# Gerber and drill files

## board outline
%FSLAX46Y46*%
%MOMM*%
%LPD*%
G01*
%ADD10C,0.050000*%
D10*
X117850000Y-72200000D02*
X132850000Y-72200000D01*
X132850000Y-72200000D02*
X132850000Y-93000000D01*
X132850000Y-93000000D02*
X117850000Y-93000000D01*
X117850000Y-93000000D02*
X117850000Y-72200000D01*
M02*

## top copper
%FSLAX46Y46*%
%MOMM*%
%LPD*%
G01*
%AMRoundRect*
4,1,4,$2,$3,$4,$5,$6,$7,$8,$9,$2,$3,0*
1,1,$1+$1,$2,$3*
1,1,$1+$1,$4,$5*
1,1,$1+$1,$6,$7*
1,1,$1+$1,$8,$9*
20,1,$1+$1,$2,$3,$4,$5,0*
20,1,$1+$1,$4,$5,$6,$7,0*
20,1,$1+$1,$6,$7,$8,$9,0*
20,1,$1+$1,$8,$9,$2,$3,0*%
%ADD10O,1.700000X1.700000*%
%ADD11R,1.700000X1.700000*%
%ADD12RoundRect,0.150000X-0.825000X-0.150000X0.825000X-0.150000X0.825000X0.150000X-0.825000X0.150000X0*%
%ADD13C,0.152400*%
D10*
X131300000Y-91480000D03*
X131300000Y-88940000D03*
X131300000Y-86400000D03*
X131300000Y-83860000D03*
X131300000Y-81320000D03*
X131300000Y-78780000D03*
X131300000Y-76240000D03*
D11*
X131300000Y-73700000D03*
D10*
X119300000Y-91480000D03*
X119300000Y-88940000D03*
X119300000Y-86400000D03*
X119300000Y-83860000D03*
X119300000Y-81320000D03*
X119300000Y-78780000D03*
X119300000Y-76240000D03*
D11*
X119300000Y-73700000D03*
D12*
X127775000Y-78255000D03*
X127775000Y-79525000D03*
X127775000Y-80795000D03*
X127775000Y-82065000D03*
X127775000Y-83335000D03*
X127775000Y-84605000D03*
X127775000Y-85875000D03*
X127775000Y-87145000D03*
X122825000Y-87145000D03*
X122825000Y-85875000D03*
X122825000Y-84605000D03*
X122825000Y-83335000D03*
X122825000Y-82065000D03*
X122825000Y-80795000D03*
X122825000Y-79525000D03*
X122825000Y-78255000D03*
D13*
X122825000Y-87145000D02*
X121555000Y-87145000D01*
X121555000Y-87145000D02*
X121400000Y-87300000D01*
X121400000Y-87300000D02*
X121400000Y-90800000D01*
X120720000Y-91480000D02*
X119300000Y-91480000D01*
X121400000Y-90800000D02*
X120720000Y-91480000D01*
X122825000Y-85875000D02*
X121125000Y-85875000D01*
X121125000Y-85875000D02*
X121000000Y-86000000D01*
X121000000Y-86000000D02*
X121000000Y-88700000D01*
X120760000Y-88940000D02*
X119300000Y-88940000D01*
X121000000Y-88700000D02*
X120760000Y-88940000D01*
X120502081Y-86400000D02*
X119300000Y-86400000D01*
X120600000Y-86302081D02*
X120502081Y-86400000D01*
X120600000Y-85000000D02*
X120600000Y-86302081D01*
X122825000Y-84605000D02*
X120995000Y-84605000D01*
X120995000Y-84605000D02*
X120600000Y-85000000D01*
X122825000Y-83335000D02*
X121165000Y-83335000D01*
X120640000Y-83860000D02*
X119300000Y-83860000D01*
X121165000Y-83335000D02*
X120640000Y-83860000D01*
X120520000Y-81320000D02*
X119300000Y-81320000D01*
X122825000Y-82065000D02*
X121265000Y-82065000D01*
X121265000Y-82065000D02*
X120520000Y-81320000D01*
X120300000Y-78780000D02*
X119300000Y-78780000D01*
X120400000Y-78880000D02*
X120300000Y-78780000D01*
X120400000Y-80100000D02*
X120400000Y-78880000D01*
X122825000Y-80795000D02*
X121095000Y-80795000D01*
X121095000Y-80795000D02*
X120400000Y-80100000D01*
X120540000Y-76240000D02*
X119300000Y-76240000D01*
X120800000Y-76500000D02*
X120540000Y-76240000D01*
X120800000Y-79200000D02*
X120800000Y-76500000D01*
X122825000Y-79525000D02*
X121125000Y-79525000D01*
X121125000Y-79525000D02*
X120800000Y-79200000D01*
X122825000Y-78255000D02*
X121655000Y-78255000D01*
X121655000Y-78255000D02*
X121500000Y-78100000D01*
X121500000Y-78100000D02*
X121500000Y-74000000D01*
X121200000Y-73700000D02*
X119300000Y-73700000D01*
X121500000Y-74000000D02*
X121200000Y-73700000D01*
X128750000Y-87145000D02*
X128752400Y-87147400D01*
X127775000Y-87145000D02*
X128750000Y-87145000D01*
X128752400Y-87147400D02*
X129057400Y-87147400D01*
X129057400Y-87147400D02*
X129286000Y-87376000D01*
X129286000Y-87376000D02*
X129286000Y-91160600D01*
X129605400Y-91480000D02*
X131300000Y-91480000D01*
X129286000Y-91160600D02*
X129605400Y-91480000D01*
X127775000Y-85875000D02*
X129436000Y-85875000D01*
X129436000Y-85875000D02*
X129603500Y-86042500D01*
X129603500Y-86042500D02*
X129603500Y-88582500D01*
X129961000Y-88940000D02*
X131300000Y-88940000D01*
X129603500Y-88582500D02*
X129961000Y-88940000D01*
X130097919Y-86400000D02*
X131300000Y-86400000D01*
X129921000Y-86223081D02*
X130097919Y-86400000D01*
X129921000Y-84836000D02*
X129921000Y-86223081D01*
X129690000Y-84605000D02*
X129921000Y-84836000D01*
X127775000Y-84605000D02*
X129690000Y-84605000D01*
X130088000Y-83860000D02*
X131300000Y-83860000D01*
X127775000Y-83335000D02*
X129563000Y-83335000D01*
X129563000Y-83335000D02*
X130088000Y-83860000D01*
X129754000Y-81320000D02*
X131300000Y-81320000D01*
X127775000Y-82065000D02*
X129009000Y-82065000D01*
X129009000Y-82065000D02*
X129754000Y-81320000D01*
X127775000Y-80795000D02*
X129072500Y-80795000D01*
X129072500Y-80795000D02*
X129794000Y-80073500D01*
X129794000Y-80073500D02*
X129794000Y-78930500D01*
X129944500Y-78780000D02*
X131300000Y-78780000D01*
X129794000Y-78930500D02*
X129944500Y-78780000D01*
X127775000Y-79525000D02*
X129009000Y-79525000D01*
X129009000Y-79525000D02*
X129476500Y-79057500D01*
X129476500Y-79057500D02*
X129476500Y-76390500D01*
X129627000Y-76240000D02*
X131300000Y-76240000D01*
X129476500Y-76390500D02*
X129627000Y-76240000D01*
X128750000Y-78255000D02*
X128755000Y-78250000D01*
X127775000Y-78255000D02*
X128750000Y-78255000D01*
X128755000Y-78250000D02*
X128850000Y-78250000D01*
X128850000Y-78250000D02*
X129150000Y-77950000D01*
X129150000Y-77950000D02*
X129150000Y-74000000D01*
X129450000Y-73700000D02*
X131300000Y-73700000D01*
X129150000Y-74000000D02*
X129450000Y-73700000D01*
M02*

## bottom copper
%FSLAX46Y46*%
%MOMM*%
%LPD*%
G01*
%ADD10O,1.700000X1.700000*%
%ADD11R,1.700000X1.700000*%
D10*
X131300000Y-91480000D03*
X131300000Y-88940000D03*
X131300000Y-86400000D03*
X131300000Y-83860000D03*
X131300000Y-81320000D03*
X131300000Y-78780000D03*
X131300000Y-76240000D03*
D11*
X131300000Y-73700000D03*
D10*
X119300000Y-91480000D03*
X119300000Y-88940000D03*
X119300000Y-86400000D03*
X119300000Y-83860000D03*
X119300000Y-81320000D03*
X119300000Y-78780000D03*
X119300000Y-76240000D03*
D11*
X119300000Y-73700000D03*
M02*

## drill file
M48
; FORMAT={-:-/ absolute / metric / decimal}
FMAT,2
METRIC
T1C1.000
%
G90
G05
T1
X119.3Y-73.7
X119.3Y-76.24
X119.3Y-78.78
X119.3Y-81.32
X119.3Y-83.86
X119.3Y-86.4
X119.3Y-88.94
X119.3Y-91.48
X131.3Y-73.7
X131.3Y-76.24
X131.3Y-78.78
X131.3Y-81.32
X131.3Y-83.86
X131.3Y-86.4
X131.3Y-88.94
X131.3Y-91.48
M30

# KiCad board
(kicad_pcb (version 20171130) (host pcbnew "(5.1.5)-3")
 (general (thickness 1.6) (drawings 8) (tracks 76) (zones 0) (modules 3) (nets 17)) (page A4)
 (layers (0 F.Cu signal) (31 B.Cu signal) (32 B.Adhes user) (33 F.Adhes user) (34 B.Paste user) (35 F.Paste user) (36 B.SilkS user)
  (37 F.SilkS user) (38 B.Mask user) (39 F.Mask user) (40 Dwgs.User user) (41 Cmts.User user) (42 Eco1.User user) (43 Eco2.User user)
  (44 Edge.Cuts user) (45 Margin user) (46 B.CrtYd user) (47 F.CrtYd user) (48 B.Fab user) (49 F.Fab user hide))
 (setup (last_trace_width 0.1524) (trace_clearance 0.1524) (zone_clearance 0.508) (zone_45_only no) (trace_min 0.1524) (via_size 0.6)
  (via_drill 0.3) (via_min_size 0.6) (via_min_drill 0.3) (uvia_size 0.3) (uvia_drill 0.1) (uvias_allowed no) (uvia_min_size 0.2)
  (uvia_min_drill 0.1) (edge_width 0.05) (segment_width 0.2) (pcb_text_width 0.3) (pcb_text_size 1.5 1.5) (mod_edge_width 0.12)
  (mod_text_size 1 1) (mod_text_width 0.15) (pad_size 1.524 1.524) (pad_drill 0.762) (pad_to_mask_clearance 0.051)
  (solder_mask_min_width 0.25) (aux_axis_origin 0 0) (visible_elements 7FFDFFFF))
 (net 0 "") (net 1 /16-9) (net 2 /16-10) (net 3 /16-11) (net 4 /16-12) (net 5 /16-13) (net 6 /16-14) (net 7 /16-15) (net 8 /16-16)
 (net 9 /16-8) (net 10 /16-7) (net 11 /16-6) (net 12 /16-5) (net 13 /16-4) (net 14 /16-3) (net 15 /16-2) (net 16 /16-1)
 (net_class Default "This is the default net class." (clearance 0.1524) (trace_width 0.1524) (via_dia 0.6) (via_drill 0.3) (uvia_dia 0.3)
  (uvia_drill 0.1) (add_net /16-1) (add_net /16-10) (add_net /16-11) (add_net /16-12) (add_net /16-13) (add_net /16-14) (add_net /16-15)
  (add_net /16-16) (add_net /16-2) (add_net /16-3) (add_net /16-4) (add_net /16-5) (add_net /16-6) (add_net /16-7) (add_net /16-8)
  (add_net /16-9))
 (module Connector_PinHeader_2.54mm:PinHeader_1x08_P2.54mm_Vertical (layer F.Cu) (at 131.3 73.7)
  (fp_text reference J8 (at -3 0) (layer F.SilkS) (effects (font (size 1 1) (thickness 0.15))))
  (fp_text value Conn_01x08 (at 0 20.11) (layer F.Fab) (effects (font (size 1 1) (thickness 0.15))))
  (pad 8 thru_hole oval (at 0 17.78) (size 1.7 1.7) (drill 1) (layers *.Cu *.Mask) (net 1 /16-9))
  (pad 7 thru_hole oval (at 0 15.24) (size 1.7 1.7) (drill 1) (layers *.Cu *.Mask) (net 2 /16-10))
  (pad 6 thru_hole oval (at 0 12.7) (size 1.7 1.7) (drill 1) (layers *.Cu *.Mask) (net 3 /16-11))
  (pad 5 thru_hole oval (at 0 10.16) (size 1.7 1.7) (drill 1) (layers *.Cu *.Mask) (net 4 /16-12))
  (pad 4 thru_hole oval (at 0 7.62) (size 1.7 1.7) (drill 1) (layers *.Cu *.Mask) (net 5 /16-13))
  (pad 3 thru_hole oval (at 0 5.08) (size 1.7 1.7) (drill 1) (layers *.Cu *.Mask) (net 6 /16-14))
  (pad 2 thru_hole oval (at 0 2.54) (size 1.7 1.7) (drill 1) (layers *.Cu *.Mask) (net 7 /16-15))
  (pad 1 thru_hole rect (at 0 0) (size 1.7 1.7) (drill 1) (layers *.Cu *.Mask) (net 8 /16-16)))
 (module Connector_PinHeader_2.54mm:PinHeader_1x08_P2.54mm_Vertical (layer F.Cu) (at 119.3 73.7)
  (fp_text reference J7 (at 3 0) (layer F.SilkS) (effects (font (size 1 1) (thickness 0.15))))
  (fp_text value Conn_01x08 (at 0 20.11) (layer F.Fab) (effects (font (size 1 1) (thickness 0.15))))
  (pad 8 thru_hole oval (at 0 17.78) (size 1.7 1.7) (drill 1) (layers *.Cu *.Mask) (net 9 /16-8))
  (pad 7 thru_hole oval (at 0 15.24) (size 1.7 1.7) (drill 1) (layers *.Cu *.Mask) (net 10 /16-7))
  (pad 6 thru_hole oval (at 0 12.7) (size 1.7 1.7) (drill 1) (layers *.Cu *.Mask) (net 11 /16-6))
  (pad 5 thru_hole oval (at 0 10.16) (size 1.7 1.7) (drill 1) (layers *.Cu *.Mask) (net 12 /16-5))
  (pad 4 thru_hole oval (at 0 7.62) (size 1.7 1.7) (drill 1) (layers *.Cu *.Mask) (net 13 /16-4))
  (pad 3 thru_hole oval (at 0 5.08) (size 1.7 1.7) (drill 1) (layers *.Cu *.Mask) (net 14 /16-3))
  (pad 2 thru_hole oval (at 0 2.54) (size 1.7 1.7) (drill 1) (layers *.Cu *.Mask) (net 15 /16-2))
  (pad 1 thru_hole rect (at 0 0) (size 1.7 1.7) (drill 1) (layers *.Cu *.Mask) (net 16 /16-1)))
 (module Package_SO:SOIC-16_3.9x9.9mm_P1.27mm (layer F.Cu) (at 125.3 82.7)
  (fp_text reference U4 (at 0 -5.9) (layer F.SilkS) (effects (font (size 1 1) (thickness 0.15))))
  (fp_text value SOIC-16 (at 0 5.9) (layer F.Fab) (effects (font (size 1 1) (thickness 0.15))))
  (pad 16 smd roundrect (at 2.475 -4.445) (size 1.95 0.6) (layers F.Cu F.Paste F.Mask) (roundrect_rratio 0.25) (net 8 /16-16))
  (pad 15 smd roundrect (at 2.475 -3.175) (size 1.95 0.6) (layers F.Cu F.Paste F.Mask) (roundrect_rratio 0.25) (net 7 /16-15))
  (pad 14 smd roundrect (at 2.475 -1.905) (size 1.95 0.6) (layers F.Cu F.Paste F.Mask) (roundrect_rratio 0.25) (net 6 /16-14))
  (pad 13 smd roundrect (at 2.475 -0.635) (size 1.95 0.6) (layers F.Cu F.Paste F.Mask) (roundrect_rratio 0.25) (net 5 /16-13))
  (pad 12 smd roundrect (at 2.475 0.635) (size 1.95 0.6) (layers F.Cu F.Paste F.Mask) (roundrect_rratio 0.25) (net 4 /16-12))
  (pad 11 smd roundrect (at 2.475 1.905) (size 1.95 0.6) (layers F.Cu F.Paste F.Mask) (roundrect_rratio 0.25) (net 3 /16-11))
  (pad 10 smd roundrect (at 2.475 3.175) (size 1.95 0.6) (layers F.Cu F.Paste F.Mask) (roundrect_rratio 0.25) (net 2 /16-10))
  (pad 9 smd roundrect (at 2.475 4.445) (size 1.95 0.6) (layers F.Cu F.Paste F.Mask) (roundrect_rratio 0.25) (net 1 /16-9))
  (pad 8 smd roundrect (at -2.475 4.445) (size 1.95 0.6) (layers F.Cu F.Paste F.Mask) (roundrect_rratio 0.25) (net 9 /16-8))
  (pad 7 smd roundrect (at -2.475 3.175) (size 1.95 0.6) (layers F.Cu F.Paste F.Mask) (roundrect_rratio 0.25) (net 10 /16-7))
  (pad 6 smd roundrect (at -2.475 1.905) (size 1.95 0.6) (layers F.Cu F.Paste F.Mask) (roundrect_rratio 0.25) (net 11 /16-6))
  (pad 5 smd roundrect (at -2.475 0.635) (size 1.95 0.6) (layers F.Cu F.Paste F.Mask) (roundrect_rratio 0.25) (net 12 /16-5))
  (pad 4 smd roundrect (at -2.475 -0.635) (size 1.95 0.6) (layers F.Cu F.Paste F.Mask) (roundrect_rratio 0.25) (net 13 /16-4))
  (pad 3 smd roundrect (at -2.475 -1.905) (size 1.95 0.6) (layers F.Cu F.Paste F.Mask) (roundrect_rratio 0.25) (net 14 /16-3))
  (pad 2 smd roundrect (at -2.475 -3.175) (size 1.95 0.6) (layers F.Cu F.Paste F.Mask) (roundrect_rratio 0.25) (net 15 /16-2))
  (pad 1 smd roundrect (at -2.475 -4.445) (size 1.95 0.6) (layers F.Cu F.Paste F.Mask) (roundrect_rratio 0.25) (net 16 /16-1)))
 (gr_line (start 117.85 72.2) (end 132.85 72.2) (layer Edge.Cuts) (width 0.05))
 (gr_line (start 132.85 72.2) (end 132.85 93) (layer Edge.Cuts) (width 0.05))
 (gr_line (start 132.85 93) (end 117.85 93) (layer Edge.Cuts) (width 0.05))
 (gr_line (start 117.85 93) (end 117.85 72.2) (layer Edge.Cuts) (width 0.05))
 (segment (start 122.825 87.145) (end 121.555 87.145) (width 0.1524) (layer F.Cu) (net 9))
 (segment (start 121.555 87.145) (end 121.4 87.3) (width 0.1524) (layer F.Cu) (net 9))
 (segment (start 121.4 87.3) (end 121.4 90.8) (width 0.1524) (layer F.Cu) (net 9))
 (segment (start 120.72 91.48) (end 119.3 91.48) (width 0.1524) (layer F.Cu) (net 9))
 (segment (start 121.4 90.8) (end 120.72 91.48) (width 0.1524) (layer F.Cu) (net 9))
 (segment (start 122.825 85.875) (end 121.125 85.875) (width 0.1524) (layer F.Cu) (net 10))
 (segment (start 121.125 85.875) (end 121 86) (width 0.1524) (layer F.Cu) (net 10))
 (segment (start 121 86) (end 121 88.7) (width 0.1524) (layer F.Cu) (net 10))
 (segment (start 120.76 88.94) (end 119.3 88.94) (width 0.1524) (layer F.Cu) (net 10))
 (segment (start 121 88.7) (end 120.76 88.94) (width 0.1524) (layer F.Cu) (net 10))
 (segment (start 120.502081 86.4) (end 119.3 86.4) (width 0.1524) (layer F.Cu) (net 11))
 (segment (start 120.6 86.302081) (end 120.502081 86.4) (width 0.1524) (layer F.Cu) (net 11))
 (segment (start 120.6 85) (end 120.6 86.302081) (width 0.1524) (layer F.Cu) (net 11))
 (segment (start 122.825 84.605) (end 120.995 84.605) (width 0.1524) (layer F.Cu) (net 11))
 (segment (start 120.995 84.605) (end 120.6 85) (width 0.1524) (layer F.Cu) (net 11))
 (segment (start 122.825 83.335) (end 121.165 83.335) (width 0.1524) (layer F.Cu) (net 12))
 (segment (start 120.64 83.86) (end 119.3 83.86) (width 0.1524) (layer F.Cu) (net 12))
 (segment (start 121.165 83.335) (end 120.64 83.86) (width 0.1524) (layer F.Cu) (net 12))
 (segment (start 120.52 81.32) (end 119.3 81.32) (width 0.1524) (layer F.Cu) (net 13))
 (segment (start 122.825 82.065) (end 121.265 82.065) (width 0.1524) (layer F.Cu) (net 13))
 (segment (start 121.265 82.065) (end 120.52 81.32) (width 0.1524) (layer F.Cu) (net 13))
 (segment (start 120.3 78.78) (end 119.3 78.78) (width 0.1524) (layer F.Cu) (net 14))
 (segment (start 120.4 78.88) (end 120.3 78.78) (width 0.1524) (layer F.Cu) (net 14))
 (segment (start 120.4 80.1) (end 120.4 78.88) (width 0.1524) (layer F.Cu) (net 14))
 (segment (start 122.825 80.795) (end 121.095 80.795) (width 0.1524) (layer F.Cu) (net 14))
 (segment (start 121.095 80.795) (end 120.4 80.1) (width 0.1524) (layer F.Cu) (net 14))
 (segment (start 120.54 76.24) (end 119.3 76.24) (width 0.1524) (layer F.Cu) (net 15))
 (segment (start 120.8 76.5) (end 120.54 76.24) (width 0.1524) (layer F.Cu) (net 15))
 (segment (start 120.8 79.2) (end 120.8 76.5) (width 0.1524) (layer F.Cu) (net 15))
 (segment (start 122.825 79.525) (end 121.125 79.525) (width 0.1524) (layer F.Cu) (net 15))
 (segment (start 121.125 79.525) (end 120.8 79.2) (width 0.1524) (layer F.Cu) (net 15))
 (segment (start 122.825 78.255) (end 121.655 78.255) (width 0.1524) (layer F.Cu) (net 16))
 (segment (start 121.655 78.255) (end 121.5 78.1) (width 0.1524) (layer F.Cu) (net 16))
 (segment (start 121.5 78.1) (end 121.5 74) (width 0.1524) (layer F.Cu) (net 16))
 (segment (start 121.2 73.7) (end 119.3 73.7) (width 0.1524) (layer F.Cu) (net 16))
 (segment (start 121.5 74) (end 121.2 73.7) (width 0.1524) (layer F.Cu) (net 16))
 (segment (start 128.75 87.145) (end 128.7524 87.1474) (width 0.1524) (layer F.Cu) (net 1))
 (segment (start 127.775 87.145) (end 128.75 87.145) (width 0.1524) (layer F.Cu) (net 1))
 (segment (start 128.7524 87.1474) (end 129.0574 87.1474) (width 0.1524) (layer F.Cu) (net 1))
 (segment (start 129.0574 87.1474) (end 129.286 87.376) (width 0.1524) (layer F.Cu) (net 1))
 (segment (start 129.286 87.376) (end 129.286 91.1606) (width 0.1524) (layer F.Cu) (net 1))
 (segment (start 129.6054 91.48) (end 131.3 91.48) (width 0.1524) (layer F.Cu) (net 1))
 (segment (start 129.286 91.1606) (end 129.6054 91.48) (width 0.1524) (layer F.Cu) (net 1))
 (segment (start 127.775 85.875) (end 129.436 85.875) (width 0.1524) (layer F.Cu) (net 2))
 (segment (start 129.436 85.875) (end 129.6035 86.0425) (width 0.1524) (layer F.Cu) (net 2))
 (segment (start 129.6035 86.0425) (end 129.6035 88.5825) (width 0.1524) (layer F.Cu) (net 2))
 (segment (start 129.961 88.94) (end 131.3 88.94) (width 0.1524) (layer F.Cu) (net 2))
 (segment (start 129.6035 88.5825) (end 129.961 88.94) (width 0.1524) (layer F.Cu) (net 2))
 (segment (start 130.097919 86.4) (end 131.3 86.4) (width 0.1524) (layer F.Cu) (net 3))
 (segment (start 129.921 86.223081) (end 130.097919 86.4) (width 0.1524) (layer F.Cu) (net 3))
 (segment (start 129.921 84.836) (end 129.921 86.223081) (width 0.1524) (layer F.Cu) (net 3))
 (segment (start 129.69 84.605) (end 129.921 84.836) (width 0.1524) (layer F.Cu) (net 3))
 (segment (start 127.775 84.605) (end 129.69 84.605) (width 0.1524) (layer F.Cu) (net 3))
 (segment (start 130.088 83.86) (end 131.3 83.86) (width 0.1524) (layer F.Cu) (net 4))
 (segment (start 127.775 83.335) (end 129.563 83.335) (width 0.1524) (layer F.Cu) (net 4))
 (segment (start 129.563 83.335) (end 130.088 83.86) (width 0.1524) (layer F.Cu) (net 4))
 (segment (start 129.754 81.32) (end 131.3 81.32) (width 0.1524) (layer F.Cu) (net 5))
 (segment (start 127.775 82.065) (end 129.009 82.065) (width 0.1524) (layer F.Cu) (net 5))
 (segment (start 129.009 82.065) (end 129.754 81.32) (width 0.1524) (layer F.Cu) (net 5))
 (segment (start 127.775 80.795) (end 129.0725 80.795) (width 0.1524) (layer F.Cu) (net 6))
 (segment (start 129.0725 80.795) (end 129.794 80.0735) (width 0.1524) (layer F.Cu) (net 6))
 (segment (start 129.794 80.0735) (end 129.794 78.9305) (width 0.1524) (layer F.Cu) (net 6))
 (segment (start 129.9445 78.78) (end 131.3 78.78) (width 0.1524) (layer F.Cu) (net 6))
 (segment (start 129.794 78.9305) (end 129.9445 78.78) (width 0.1524) (layer F.Cu) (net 6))
 (segment (start 127.775 79.525) (end 129.009 79.525) (width 0.1524) (layer F.Cu) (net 7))
 (segment (start 129.009 79.525) (end 129.4765 79.0575) (width 0.1524) (layer F.Cu) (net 7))
 (segment (start 129.4765 79.0575) (end 129.4765 76.3905) (width 0.1524) (layer F.Cu) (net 7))
 (segment (start 129.627 76.24) (end 131.3 76.24) (width 0.1524) (layer F.Cu) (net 7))
 (segment (start 129.4765 76.3905) (end 129.627 76.24) (width 0.1524) (layer F.Cu) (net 7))
 (segment (start 128.75 78.255) (end 128.755 78.25) (width 0.1524) (layer F.Cu) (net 8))
 (segment (start 127.775 78.255) (end 128.75 78.255) (width 0.1524) (layer F.Cu) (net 8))
 (segment (start 128.755 78.25) (end 128.85 78.25) (width 0.1524) (layer F.Cu) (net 8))
 (segment (start 128.85 78.25) (end 129.15 77.95) (width 0.1524) (layer F.Cu) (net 8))
 (segment (start 129.15 77.95) (end 129.15 74) (width 0.1524) (layer F.Cu) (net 8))
 (segment (start 129.45 73.7) (end 131.3 73.7) (width 0.1524) (layer F.Cu) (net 8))
 (segment (start 129.15 74) (end 129.45 73.7) (width 0.1524) (layer F.Cu) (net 8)))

